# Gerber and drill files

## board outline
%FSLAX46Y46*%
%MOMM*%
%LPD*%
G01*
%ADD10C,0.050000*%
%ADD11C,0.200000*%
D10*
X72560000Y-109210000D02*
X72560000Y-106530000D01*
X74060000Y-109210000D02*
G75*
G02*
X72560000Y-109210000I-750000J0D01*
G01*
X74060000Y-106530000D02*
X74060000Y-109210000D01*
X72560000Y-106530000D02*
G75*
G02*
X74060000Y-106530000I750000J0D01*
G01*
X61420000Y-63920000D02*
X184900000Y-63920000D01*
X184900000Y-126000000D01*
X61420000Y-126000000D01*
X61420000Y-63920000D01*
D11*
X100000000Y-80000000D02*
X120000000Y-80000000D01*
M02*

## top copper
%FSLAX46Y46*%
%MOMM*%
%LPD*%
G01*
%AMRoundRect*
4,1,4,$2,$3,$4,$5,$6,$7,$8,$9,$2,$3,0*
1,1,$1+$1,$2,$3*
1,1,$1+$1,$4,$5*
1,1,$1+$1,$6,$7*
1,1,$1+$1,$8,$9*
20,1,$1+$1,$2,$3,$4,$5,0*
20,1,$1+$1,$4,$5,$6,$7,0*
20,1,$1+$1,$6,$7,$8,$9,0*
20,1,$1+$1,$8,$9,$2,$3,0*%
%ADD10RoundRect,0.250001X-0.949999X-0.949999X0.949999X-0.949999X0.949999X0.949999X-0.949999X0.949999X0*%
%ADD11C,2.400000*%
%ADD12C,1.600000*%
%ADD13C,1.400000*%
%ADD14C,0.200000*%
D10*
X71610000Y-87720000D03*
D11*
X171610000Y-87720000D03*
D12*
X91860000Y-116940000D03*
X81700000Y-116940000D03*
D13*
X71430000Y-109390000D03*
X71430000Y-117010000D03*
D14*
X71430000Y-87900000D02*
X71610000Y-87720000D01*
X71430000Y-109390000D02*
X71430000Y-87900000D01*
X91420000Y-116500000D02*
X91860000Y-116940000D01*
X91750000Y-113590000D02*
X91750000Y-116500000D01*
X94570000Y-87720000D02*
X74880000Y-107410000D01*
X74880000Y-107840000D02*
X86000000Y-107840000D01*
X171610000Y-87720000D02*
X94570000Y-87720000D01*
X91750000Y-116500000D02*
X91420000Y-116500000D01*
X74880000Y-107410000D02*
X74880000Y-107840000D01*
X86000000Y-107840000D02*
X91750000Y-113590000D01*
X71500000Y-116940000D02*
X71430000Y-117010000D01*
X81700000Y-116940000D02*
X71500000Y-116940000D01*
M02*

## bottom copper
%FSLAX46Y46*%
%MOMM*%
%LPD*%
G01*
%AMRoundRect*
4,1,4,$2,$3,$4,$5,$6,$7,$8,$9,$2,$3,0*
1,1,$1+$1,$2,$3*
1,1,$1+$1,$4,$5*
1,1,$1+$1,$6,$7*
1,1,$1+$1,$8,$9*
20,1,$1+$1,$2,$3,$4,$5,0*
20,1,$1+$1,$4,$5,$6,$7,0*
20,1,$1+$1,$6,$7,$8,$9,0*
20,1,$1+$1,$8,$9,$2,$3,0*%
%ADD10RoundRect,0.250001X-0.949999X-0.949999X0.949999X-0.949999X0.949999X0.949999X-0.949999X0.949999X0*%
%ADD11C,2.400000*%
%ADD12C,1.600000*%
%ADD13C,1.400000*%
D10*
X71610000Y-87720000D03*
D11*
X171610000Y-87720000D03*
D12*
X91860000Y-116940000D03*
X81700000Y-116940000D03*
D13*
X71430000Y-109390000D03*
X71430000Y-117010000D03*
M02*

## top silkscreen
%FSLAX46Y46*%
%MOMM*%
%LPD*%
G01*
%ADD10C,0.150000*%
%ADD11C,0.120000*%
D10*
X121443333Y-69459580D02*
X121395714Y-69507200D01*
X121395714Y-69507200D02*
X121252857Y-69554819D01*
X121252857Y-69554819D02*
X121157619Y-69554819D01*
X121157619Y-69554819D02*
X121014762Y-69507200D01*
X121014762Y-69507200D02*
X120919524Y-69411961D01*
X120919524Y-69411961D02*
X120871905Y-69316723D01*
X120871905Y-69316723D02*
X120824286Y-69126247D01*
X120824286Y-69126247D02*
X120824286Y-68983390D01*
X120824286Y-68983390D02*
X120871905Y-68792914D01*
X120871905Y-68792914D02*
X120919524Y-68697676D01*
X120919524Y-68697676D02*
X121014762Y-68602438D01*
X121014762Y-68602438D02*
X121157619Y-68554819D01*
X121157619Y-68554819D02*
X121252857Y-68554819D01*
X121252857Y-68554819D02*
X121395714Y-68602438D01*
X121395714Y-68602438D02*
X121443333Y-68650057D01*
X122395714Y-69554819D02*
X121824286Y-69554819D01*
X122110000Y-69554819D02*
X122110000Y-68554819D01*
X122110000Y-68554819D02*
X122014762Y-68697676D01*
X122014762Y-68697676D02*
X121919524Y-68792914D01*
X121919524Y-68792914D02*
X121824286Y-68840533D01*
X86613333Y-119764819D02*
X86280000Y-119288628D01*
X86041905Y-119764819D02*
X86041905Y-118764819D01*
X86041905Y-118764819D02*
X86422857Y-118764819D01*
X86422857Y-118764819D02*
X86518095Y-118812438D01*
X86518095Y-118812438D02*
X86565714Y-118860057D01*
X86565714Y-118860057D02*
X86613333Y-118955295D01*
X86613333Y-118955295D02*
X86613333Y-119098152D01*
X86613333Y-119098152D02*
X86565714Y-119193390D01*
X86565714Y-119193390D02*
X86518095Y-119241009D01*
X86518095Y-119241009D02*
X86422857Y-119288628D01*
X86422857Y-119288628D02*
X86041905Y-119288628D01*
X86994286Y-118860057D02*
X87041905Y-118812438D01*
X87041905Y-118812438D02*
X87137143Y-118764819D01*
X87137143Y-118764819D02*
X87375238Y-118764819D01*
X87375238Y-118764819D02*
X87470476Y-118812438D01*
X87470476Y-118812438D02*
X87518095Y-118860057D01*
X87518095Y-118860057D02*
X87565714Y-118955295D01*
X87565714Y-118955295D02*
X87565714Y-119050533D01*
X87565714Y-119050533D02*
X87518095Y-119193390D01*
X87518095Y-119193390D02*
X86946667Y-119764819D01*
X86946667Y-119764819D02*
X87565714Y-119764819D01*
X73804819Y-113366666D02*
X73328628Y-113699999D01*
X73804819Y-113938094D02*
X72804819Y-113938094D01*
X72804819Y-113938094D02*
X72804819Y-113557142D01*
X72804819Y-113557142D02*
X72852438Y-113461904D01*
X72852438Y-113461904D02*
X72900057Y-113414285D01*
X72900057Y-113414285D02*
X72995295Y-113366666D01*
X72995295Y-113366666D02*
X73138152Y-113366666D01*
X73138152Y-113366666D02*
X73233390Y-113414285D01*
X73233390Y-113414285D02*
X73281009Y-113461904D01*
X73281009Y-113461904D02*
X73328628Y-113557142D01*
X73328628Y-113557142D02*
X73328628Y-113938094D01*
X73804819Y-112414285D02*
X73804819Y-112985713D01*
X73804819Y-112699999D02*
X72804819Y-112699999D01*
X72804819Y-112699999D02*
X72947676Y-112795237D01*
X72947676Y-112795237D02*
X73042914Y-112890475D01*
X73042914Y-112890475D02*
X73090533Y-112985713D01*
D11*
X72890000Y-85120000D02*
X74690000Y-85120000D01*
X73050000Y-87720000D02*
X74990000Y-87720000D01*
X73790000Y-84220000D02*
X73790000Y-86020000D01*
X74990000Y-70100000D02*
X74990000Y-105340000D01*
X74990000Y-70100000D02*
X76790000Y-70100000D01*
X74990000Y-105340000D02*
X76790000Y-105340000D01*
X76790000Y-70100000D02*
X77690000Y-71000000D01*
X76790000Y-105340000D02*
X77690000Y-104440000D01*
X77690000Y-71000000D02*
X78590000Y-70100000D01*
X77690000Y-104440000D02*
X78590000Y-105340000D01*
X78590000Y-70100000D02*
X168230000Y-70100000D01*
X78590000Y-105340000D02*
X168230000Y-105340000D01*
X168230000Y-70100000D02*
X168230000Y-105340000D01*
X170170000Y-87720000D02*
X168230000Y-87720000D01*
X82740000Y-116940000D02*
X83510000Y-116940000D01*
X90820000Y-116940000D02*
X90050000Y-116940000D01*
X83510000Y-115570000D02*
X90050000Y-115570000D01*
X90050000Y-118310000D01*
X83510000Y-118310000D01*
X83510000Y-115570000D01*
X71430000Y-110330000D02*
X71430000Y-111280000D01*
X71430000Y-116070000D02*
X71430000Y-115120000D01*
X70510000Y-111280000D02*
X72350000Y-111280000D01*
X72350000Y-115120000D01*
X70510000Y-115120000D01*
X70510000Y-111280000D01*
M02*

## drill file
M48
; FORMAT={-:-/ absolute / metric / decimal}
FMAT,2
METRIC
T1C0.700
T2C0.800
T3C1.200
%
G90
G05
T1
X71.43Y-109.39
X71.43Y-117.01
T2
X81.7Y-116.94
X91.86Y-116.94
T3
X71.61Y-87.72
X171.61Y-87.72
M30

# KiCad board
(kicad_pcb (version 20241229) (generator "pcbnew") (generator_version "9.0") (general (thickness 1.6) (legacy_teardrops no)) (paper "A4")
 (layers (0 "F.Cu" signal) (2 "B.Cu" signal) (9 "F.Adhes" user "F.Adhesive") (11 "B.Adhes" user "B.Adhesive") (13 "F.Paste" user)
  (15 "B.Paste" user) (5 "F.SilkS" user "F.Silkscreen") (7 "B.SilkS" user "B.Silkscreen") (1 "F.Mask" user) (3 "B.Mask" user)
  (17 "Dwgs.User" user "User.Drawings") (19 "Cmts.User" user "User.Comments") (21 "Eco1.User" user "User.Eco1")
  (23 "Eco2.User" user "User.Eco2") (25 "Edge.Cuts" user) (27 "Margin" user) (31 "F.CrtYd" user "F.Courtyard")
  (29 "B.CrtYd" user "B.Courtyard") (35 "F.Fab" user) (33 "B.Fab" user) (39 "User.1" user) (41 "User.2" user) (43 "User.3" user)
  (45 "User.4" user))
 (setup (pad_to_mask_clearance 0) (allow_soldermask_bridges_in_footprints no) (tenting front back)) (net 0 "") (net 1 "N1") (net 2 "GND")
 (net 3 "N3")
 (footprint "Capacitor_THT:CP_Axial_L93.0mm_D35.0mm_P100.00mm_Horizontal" (layer "F.Cu") (at 71.61 87.72)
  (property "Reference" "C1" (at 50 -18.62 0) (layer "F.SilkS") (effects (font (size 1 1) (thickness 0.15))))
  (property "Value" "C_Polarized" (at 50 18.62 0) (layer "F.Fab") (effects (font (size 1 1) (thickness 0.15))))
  (fp_line (start 1.28 -2.6) (end 3.08 -2.6) (stroke (width 0.12) (type solid)) (layer "F.SilkS"))
  (fp_line (start 1.44 0) (end 3.38 0) (stroke (width 0.12) (type solid)) (layer "F.SilkS"))
  (fp_line (start 2.18 -3.5) (end 2.18 -1.7) (stroke (width 0.12) (type solid)) (layer "F.SilkS"))
  (fp_line (start 3.38 -17.62) (end 3.38 17.62) (stroke (width 0.12) (type solid)) (layer "F.SilkS"))
  (fp_line (start 3.38 -17.62) (end 5.18 -17.62) (stroke (width 0.12) (type solid)) (layer "F.SilkS"))
  (fp_line (start 3.38 17.62) (end 5.18 17.62) (stroke (width 0.12) (type solid)) (layer "F.SilkS"))
  (fp_line (start 5.18 -17.62) (end 6.08 -16.72) (stroke (width 0.12) (type solid)) (layer "F.SilkS"))
  (fp_line (start 5.18 17.62) (end 6.08 16.72) (stroke (width 0.12) (type solid)) (layer "F.SilkS"))
  (fp_line (start 6.08 -16.72) (end 6.98 -17.62) (stroke (width 0.12) (type solid)) (layer "F.SilkS"))
  (fp_line (start 6.08 16.72) (end 6.98 17.62) (stroke (width 0.12) (type solid)) (layer "F.SilkS"))
  (fp_line (start 6.98 -17.62) (end 96.62 -17.62) (stroke (width 0.12) (type solid)) (layer "F.SilkS"))
  (fp_line (start 6.98 17.62) (end 96.62 17.62) (stroke (width 0.12) (type solid)) (layer "F.SilkS"))
  (fp_line (start 96.62 -17.62) (end 96.62 17.62) (stroke (width 0.12) (type solid)) (layer "F.SilkS"))
  (fp_line (start 98.56 0) (end 96.62 0) (stroke (width 0.12) (type solid)) (layer "F.SilkS"))
  (pad "1" thru_hole roundrect (at 0 0) (size 2.4 2.4) (drill 1.2) (layers "*.Cu" "*.Mask") (remove_unused_layers no)
   (roundrect_rratio 0.104167) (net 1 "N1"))
  (pad "2" thru_hole circle (at 100 0) (size 2.4 2.4) (drill 1.2) (layers "*.Cu" "*.Mask") (remove_unused_layers no) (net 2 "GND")))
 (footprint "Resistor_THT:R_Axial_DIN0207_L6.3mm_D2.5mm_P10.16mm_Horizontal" (layer "F.Cu") (at 91.86 116.94 180)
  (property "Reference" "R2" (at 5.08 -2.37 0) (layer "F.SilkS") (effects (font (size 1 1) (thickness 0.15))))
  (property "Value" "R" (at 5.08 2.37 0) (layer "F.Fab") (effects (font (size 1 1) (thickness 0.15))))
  (fp_line (start 9.12 0) (end 8.35 0) (stroke (width 0.12) (type solid)) (layer "F.SilkS"))
  (fp_line (start 1.04 0) (end 1.81 0) (stroke (width 0.12) (type solid)) (layer "F.SilkS"))
  (fp_rect (start 1.81 -1.37) (end 8.35 1.37) (stroke (width 0.12) (type solid)) (fill no) (layer "F.SilkS"))
  (pad "1" thru_hole circle (at 0 0 180) (size 1.6 1.6) (drill 0.8) (layers "*.Cu" "*.Mask") (remove_unused_layers no) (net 2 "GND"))
  (pad "2" thru_hole circle (at 10.16 0 180) (size 1.6 1.6) (drill 0.8) (layers "*.Cu" "*.Mask") (remove_unused_layers no) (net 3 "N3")))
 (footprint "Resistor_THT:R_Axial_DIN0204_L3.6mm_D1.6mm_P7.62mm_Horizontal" (layer "F.Cu") (at 71.43 109.39 -90)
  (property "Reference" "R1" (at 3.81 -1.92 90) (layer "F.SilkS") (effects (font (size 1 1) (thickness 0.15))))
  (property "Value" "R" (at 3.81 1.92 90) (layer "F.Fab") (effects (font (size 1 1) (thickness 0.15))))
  (fp_line (start 0.94 0) (end 1.89 0) (stroke (width 0.12) (type solid)) (layer "F.SilkS"))
  (fp_line (start 6.68 0) (end 5.73 0) (stroke (width 0.12) (type solid)) (layer "F.SilkS"))
  (fp_rect (start 1.89 -0.92) (end 5.73 0.92) (stroke (width 0.12) (type solid)) (fill no) (layer "F.SilkS"))
  (pad "1" thru_hole circle (at 0 0 270) (size 1.4 1.4) (drill 0.7) (layers "*.Cu" "*.Mask") (remove_unused_layers no) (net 1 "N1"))
  (pad "2" thru_hole circle (at 7.62 0 270) (size 1.4 1.4) (drill 0.7) (layers "*.Cu" "*.Mask") (remove_unused_layers no) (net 3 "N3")))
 (gr_line (start 72.56 109.21) (end 72.56 106.53) (stroke (width 0.05) (type default)) (layer "Edge.Cuts"))
 (gr_arc (start 74.06 109.21) (mid 73.31 109.96) (end 72.56 109.21) (stroke (width 0.05) (type default)) (layer "Edge.Cuts"))
 (gr_line (start 74.06 106.53) (end 74.06 109.21) (stroke (width 0.05) (type default)) (layer "Edge.Cuts"))
 (gr_arc (start 72.56 106.53) (mid 73.31 105.78) (end 74.06 106.53) (stroke (width 0.05) (type default)) (layer "Edge.Cuts"))
 (gr_rect (start 61.42 63.92) (end 184.9 126) (stroke (width 0.05) (type default)) (fill no) (layer "Edge.Cuts"))
 (segment (start 71.43 87.9) (end 71.61 87.72) (width 0.2) (layer "F.Cu") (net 1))
 (segment (start 71.43 109.39) (end 71.43 87.9) (width 0.2) (layer "F.Cu") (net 1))
 (segment (start 91.42 116.5) (end 91.86 116.94) (width 0.2) (layer "F.Cu") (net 2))
 (segment (start 91.75 113.59) (end 91.75 116.5) (width 0.2) (layer "F.Cu") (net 2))
 (segment (start 94.57 87.72) (end 74.88 107.41) (width 0.2) (layer "F.Cu") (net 2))
 (segment (start 74.88 107.84) (end 86 107.84) (width 0.2) (layer "F.Cu") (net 2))
 (segment (start 171.61 87.72) (end 94.57 87.72) (width 0.2) (layer "F.Cu") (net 2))
 (segment (start 91.75 116.5) (end 91.42 116.5) (width 0.2) (layer "F.Cu") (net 2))
 (segment (start 74.88 107.41) (end 74.88 107.84) (width 0.2) (layer "F.Cu") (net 2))
 (segment (start 86 107.84) (end 91.75 113.59) (width 0.2) (layer "F.Cu") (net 2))
 (segment (start 71.5 116.94) (end 71.43 117.01) (width 0.2) (layer "F.Cu") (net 3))
 (segment (start 81.7 116.94) (end 71.5 116.94) (width 0.2) (layer "F.Cu") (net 3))
 (gr_line (start 100 80) (end 120 80) (stroke (width 0.2) (type solid)) (layer "Edge.Cuts")))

